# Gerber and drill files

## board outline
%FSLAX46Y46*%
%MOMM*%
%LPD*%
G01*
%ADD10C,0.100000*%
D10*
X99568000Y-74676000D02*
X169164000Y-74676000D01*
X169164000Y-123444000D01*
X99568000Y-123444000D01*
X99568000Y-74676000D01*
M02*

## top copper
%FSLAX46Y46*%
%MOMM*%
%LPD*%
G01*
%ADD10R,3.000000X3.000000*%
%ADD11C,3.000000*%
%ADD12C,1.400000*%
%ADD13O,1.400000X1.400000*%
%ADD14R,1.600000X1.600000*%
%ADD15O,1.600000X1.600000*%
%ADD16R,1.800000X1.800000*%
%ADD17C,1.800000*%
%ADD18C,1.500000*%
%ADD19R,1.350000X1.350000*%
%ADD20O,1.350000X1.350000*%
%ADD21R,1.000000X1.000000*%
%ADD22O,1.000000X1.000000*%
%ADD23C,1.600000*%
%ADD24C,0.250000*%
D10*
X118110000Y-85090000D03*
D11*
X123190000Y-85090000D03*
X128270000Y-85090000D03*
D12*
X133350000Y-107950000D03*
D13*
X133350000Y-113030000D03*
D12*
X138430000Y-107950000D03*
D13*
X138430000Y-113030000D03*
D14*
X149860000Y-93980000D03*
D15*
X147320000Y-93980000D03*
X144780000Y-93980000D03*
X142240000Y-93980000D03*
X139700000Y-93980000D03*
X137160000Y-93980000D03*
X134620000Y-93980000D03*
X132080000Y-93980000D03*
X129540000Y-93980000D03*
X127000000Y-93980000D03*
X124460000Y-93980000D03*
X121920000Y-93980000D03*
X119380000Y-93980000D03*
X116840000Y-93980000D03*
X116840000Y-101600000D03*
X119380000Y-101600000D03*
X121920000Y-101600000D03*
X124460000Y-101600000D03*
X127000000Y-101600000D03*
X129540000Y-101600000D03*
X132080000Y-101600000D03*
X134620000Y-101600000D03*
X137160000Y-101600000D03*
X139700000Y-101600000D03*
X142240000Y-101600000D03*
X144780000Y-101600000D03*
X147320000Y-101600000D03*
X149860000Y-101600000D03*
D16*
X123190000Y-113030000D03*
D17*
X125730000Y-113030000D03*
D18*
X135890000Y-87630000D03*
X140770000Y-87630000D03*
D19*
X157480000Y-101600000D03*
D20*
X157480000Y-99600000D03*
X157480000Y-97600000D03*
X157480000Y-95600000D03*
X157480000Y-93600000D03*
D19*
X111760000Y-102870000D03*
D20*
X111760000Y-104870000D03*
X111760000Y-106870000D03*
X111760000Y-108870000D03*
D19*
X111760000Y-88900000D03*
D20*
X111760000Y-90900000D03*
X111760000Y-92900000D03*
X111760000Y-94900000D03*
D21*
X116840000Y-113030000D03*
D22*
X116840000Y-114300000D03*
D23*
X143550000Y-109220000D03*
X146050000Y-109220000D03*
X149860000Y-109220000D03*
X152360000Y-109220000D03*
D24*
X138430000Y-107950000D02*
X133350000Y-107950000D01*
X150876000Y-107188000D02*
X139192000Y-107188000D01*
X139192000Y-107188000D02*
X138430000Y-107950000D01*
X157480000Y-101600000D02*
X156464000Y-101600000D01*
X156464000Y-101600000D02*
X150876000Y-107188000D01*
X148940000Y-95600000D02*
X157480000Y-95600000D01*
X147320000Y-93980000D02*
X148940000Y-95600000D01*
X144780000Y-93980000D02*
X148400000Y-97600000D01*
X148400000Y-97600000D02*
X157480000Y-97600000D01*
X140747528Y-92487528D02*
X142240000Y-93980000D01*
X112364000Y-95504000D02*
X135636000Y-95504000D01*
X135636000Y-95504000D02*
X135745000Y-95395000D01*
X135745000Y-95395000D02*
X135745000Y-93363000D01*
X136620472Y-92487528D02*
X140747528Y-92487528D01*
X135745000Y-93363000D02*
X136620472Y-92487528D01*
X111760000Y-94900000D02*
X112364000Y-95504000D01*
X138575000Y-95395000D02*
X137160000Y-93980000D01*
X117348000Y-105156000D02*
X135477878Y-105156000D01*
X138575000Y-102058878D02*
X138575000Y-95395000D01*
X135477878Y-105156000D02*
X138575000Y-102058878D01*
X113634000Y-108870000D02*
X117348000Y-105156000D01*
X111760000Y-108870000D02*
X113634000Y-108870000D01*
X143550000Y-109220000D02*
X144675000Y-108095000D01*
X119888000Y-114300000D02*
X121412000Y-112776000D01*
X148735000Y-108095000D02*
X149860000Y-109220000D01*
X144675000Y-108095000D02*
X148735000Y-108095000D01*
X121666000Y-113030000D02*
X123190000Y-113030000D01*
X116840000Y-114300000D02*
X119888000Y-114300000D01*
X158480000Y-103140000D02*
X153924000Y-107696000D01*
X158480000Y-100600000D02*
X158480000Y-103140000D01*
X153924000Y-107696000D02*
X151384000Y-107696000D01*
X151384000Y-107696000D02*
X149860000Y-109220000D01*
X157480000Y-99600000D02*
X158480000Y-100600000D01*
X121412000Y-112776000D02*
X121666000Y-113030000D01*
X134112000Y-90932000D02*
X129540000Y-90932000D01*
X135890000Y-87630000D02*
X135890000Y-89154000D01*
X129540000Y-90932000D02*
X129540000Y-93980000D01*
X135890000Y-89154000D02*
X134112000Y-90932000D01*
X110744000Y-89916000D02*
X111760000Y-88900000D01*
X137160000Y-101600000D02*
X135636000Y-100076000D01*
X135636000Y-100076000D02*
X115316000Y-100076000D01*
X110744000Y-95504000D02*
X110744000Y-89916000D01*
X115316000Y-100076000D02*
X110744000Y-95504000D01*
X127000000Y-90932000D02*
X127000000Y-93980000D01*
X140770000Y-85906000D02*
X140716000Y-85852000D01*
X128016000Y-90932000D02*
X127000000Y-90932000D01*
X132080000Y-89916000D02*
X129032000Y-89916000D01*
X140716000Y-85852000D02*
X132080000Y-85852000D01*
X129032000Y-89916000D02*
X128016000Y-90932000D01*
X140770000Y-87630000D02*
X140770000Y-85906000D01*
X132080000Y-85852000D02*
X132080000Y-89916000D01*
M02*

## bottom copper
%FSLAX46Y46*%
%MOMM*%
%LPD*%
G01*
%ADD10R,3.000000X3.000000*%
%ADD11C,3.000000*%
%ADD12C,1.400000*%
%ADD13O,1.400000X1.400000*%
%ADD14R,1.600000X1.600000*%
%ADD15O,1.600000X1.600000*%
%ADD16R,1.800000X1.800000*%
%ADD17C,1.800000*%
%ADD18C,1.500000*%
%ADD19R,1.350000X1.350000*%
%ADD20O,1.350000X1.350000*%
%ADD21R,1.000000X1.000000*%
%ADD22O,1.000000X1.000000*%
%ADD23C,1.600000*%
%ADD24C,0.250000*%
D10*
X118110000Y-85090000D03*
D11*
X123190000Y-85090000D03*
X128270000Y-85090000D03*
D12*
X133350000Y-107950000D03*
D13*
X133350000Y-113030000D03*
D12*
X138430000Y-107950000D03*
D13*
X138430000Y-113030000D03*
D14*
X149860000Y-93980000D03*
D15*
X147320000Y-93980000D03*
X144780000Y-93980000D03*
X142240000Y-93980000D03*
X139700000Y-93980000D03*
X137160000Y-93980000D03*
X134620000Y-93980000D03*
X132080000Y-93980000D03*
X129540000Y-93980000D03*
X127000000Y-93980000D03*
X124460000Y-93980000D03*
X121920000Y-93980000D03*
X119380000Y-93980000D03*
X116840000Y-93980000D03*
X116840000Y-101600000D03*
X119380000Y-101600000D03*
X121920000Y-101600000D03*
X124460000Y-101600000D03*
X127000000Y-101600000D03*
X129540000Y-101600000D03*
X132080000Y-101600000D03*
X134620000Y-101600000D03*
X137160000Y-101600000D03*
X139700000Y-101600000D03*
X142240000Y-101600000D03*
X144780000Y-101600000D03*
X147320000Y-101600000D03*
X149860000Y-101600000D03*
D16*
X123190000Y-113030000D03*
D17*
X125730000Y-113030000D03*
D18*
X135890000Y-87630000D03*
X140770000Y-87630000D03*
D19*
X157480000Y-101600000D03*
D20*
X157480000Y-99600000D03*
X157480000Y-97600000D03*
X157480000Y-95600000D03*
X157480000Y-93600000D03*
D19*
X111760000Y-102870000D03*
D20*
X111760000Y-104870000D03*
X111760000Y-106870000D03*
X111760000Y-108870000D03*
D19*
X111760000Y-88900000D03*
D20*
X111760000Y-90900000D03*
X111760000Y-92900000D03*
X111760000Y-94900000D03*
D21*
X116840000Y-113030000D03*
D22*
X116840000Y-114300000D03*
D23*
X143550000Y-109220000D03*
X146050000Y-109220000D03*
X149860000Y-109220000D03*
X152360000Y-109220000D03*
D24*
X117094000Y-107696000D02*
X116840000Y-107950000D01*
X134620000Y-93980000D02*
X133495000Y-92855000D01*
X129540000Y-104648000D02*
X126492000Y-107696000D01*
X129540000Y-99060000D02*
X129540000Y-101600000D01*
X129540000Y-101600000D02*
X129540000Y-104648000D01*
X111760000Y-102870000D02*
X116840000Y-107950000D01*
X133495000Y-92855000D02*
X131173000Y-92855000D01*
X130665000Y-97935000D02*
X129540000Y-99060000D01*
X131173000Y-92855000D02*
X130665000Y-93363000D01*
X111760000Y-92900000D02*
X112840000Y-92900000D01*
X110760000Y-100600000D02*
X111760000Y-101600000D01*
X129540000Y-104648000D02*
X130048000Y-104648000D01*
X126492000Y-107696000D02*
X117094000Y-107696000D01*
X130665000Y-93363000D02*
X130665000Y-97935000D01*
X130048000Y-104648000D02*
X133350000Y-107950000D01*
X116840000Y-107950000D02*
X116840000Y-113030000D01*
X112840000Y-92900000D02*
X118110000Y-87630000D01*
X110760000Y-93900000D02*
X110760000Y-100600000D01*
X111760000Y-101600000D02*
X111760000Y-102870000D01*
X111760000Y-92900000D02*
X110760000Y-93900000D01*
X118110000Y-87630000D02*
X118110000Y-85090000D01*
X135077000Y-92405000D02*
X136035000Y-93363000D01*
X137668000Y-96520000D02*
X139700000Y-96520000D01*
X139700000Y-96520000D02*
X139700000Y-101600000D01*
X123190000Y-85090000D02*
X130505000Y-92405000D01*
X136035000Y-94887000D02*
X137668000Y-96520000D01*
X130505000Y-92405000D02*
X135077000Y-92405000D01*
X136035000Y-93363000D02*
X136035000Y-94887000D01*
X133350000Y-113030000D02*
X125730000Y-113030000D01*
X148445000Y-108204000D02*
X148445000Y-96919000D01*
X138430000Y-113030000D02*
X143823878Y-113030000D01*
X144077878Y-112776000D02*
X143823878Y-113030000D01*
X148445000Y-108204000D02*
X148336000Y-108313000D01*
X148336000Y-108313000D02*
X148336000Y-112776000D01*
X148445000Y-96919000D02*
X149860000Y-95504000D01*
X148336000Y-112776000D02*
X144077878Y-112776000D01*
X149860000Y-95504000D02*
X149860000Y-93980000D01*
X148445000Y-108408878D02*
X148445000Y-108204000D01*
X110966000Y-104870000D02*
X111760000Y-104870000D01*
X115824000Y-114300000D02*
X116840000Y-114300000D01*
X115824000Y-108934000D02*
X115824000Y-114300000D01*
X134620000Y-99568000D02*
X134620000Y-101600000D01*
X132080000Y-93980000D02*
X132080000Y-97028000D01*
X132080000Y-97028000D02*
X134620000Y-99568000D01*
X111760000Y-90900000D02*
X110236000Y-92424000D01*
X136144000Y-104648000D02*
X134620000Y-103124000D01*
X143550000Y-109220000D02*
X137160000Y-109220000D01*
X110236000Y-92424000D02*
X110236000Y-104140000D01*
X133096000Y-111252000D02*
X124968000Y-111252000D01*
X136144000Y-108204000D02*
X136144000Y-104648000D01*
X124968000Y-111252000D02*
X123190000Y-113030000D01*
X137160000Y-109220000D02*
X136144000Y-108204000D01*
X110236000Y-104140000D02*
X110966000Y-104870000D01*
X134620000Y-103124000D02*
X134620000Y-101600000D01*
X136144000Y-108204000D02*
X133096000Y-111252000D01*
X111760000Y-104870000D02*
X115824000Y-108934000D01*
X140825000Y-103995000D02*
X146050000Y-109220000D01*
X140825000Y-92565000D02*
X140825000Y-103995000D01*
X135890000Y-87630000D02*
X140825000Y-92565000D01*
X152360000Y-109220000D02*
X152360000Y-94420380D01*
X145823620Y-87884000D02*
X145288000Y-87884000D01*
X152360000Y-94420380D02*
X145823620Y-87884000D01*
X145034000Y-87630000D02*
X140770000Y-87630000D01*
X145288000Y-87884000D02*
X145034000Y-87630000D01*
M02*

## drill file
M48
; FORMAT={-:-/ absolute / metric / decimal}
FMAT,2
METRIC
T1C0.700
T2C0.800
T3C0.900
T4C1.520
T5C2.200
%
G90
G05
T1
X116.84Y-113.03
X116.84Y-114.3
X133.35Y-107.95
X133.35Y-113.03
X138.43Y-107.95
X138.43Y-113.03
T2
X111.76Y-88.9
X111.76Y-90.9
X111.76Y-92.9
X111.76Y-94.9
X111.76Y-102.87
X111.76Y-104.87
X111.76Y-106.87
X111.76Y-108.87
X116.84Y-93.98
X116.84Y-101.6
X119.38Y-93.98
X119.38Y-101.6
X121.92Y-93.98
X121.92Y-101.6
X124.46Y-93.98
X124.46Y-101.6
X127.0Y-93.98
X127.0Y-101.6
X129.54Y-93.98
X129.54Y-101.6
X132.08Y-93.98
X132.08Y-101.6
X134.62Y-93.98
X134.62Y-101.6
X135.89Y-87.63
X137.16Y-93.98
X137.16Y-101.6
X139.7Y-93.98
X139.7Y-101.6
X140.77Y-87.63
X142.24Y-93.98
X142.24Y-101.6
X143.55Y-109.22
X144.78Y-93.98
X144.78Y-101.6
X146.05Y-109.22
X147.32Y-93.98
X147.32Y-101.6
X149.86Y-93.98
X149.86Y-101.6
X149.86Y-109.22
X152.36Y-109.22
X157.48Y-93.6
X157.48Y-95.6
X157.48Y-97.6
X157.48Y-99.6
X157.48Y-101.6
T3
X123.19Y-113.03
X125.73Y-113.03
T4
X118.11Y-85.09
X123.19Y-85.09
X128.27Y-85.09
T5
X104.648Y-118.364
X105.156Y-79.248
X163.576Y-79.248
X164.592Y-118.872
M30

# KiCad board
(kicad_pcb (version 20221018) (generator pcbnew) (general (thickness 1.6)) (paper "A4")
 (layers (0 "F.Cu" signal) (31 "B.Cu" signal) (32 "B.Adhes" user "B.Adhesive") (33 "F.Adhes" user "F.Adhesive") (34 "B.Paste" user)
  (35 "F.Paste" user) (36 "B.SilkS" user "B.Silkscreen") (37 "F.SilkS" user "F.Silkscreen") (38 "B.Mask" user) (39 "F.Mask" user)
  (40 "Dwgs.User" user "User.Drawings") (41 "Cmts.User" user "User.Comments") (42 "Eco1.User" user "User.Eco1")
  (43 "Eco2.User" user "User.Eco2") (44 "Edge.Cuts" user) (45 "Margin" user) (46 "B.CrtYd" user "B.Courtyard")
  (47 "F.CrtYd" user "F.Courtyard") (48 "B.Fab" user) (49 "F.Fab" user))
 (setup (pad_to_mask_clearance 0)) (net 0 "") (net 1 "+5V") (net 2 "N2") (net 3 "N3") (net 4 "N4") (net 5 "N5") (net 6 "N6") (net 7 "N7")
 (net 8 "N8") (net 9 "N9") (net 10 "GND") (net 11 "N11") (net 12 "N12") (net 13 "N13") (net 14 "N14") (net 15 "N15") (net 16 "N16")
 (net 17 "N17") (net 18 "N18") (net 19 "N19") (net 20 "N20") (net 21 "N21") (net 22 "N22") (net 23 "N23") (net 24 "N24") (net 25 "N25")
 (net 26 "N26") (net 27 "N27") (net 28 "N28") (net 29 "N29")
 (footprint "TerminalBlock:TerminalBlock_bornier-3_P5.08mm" (layer "F.Cu") (at 118.11 85.09)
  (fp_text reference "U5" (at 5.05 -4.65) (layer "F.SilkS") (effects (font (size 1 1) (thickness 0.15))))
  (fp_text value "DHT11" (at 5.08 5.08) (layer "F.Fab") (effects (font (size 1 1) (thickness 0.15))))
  (pad "1" thru_hole rect (at 0 0) (size 3 3) (drill 1.52) (layers "*.Cu" "*.Mask") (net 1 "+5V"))
  (pad "2" thru_hole circle (at 5.08 0) (size 3 3) (drill 1.52) (layers "*.Cu" "*.Mask") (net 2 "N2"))
  (pad "3" thru_hole circle (at 10.16 0) (size 3 3) (drill 1.52) (layers "*.Cu" "*.Mask")))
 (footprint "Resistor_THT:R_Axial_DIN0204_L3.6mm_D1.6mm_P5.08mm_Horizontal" (layer "F.Cu") (at 133.35 107.95 -90)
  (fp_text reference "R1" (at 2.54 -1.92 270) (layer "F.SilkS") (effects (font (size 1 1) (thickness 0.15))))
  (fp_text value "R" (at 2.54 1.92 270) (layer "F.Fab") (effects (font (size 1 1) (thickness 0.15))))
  (pad "1" thru_hole circle (at 0 0 270) (size 1.4 1.4) (drill 0.7) (layers "*.Cu" "*.Mask") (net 1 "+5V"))
  (pad "2" thru_hole oval (at 5.08 0 270) (size 1.4 1.4) (drill 0.7) (layers "*.Cu" "*.Mask") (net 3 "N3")))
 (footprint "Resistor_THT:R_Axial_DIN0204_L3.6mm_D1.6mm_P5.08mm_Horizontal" (layer "F.Cu") (at 138.43 107.95 -90)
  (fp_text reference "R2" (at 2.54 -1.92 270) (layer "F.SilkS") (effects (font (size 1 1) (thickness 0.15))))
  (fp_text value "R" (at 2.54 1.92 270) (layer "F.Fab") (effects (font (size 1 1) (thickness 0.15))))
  (pad "1" thru_hole circle (at 0 0 270) (size 1.4 1.4) (drill 0.7) (layers "*.Cu" "*.Mask") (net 1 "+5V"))
  (pad "2" thru_hole oval (at 5.08 0 270) (size 1.4 1.4) (drill 0.7) (layers "*.Cu" "*.Mask") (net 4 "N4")))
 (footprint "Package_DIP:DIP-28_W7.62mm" (layer "F.Cu") (at 149.86 93.98 -90)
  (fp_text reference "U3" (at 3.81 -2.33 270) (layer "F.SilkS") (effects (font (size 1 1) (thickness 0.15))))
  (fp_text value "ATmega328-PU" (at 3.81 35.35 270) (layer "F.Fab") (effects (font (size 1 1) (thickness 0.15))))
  (pad "1" thru_hole rect (at 0 0 270) (size 1.6 1.6) (drill 0.8) (layers "*.Cu" "*.Mask") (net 4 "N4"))
  (pad "2" thru_hole oval (at 0 2.54 270) (size 1.6 1.6) (drill 0.8) (layers "*.Cu" "*.Mask") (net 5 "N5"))
  (pad "3" thru_hole oval (at 0 5.08 270) (size 1.6 1.6) (drill 0.8) (layers "*.Cu" "*.Mask") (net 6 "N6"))
  (pad "4" thru_hole oval (at 0 7.62 270) (size 1.6 1.6) (drill 0.8) (layers "*.Cu" "*.Mask") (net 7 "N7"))
  (pad "5" thru_hole oval (at 0 10.16 270) (size 1.6 1.6) (drill 0.8) (layers "*.Cu" "*.Mask") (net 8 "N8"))
  (pad "6" thru_hole oval (at 0 12.7 270) (size 1.6 1.6) (drill 0.8) (layers "*.Cu" "*.Mask") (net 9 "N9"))
  (pad "7" thru_hole oval (at 0 15.24 270) (size 1.6 1.6) (drill 0.8) (layers "*.Cu" "*.Mask") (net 1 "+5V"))
  (pad "8" thru_hole oval (at 0 17.78 270) (size 1.6 1.6) (drill 0.8) (layers "*.Cu" "*.Mask") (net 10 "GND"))
  (pad "9" thru_hole oval (at 0 20.32 270) (size 1.6 1.6) (drill 0.8) (layers "*.Cu" "*.Mask") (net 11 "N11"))
  (pad "10" thru_hole oval (at 0 22.86 270) (size 1.6 1.6) (drill 0.8) (layers "*.Cu" "*.Mask") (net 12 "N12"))
  (pad "11" thru_hole oval (at 0 25.4 270) (size 1.6 1.6) (drill 0.8) (layers "*.Cu" "*.Mask") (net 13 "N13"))
  (pad "12" thru_hole oval (at 0 27.94 270) (size 1.6 1.6) (drill 0.8) (layers "*.Cu" "*.Mask") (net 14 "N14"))
  (pad "13" thru_hole oval (at 0 30.48 270) (size 1.6 1.6) (drill 0.8) (layers "*.Cu" "*.Mask") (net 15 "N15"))
  (pad "14" thru_hole oval (at 0 33.02 270) (size 1.6 1.6) (drill 0.8) (layers "*.Cu" "*.Mask") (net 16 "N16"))
  (pad "15" thru_hole oval (at 7.62 33.02 270) (size 1.6 1.6) (drill 0.8) (layers "*.Cu" "*.Mask") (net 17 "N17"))
  (pad "16" thru_hole oval (at 7.62 30.48 270) (size 1.6 1.6) (drill 0.8) (layers "*.Cu" "*.Mask") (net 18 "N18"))
  (pad "17" thru_hole oval (at 7.62 27.94 270) (size 1.6 1.6) (drill 0.8) (layers "*.Cu" "*.Mask") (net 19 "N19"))
  (pad "18" thru_hole oval (at 7.62 25.4 270) (size 1.6 1.6) (drill 0.8) (layers "*.Cu" "*.Mask") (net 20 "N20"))
  (pad "19" thru_hole oval (at 7.62 22.86 270) (size 1.6 1.6) (drill 0.8) (layers "*.Cu" "*.Mask") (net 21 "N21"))
  (pad "20" thru_hole oval (at 7.62 20.32 270) (size 1.6 1.6) (drill 0.8) (layers "*.Cu" "*.Mask") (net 1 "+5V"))
  (pad "21" thru_hole oval (at 7.62 17.78 270) (size 1.6 1.6) (drill 0.8) (layers "*.Cu" "*.Mask") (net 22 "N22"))
  (pad "22" thru_hole oval (at 7.62 15.24 270) (size 1.6 1.6) (drill 0.8) (layers "*.Cu" "*.Mask") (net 10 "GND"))
  (pad "23" thru_hole oval (at 7.62 12.7 270) (size 1.6 1.6) (drill 0.8) (layers "*.Cu" "*.Mask") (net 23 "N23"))
  (pad "24" thru_hole oval (at 7.62 10.16 270) (size 1.6 1.6) (drill 0.8) (layers "*.Cu" "*.Mask") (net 2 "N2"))
  (pad "25" thru_hole oval (at 7.62 7.62 270) (size 1.6 1.6) (drill 0.8) (layers "*.Cu" "*.Mask") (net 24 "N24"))
  (pad "26" thru_hole oval (at 7.62 5.08 270) (size 1.6 1.6) (drill 0.8) (layers "*.Cu" "*.Mask") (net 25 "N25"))
  (pad "27" thru_hole oval (at 7.62 2.54 270) (size 1.6 1.6) (drill 0.8) (layers "*.Cu" "*.Mask") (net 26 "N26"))
  (pad "28" thru_hole oval (at 7.62 0 270) (size 1.6 1.6) (drill 0.8) (layers "*.Cu" "*.Mask") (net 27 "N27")))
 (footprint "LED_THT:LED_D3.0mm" (layer "F.Cu") (at 123.19 113.03)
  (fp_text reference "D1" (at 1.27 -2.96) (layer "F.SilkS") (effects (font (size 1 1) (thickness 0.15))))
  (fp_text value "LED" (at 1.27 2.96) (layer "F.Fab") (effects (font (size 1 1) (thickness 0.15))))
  (pad "1" thru_hole rect (at 0 0) (size 1.8 1.8) (drill 0.9) (layers "*.Cu" "*.Mask") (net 10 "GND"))
  (pad "2" thru_hole circle (at 2.54 0) (size 1.8 1.8) (drill 0.9) (layers "*.Cu" "*.Mask") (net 3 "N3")))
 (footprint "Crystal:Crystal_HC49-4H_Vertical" (layer "F.Cu") (at 135.89 87.63)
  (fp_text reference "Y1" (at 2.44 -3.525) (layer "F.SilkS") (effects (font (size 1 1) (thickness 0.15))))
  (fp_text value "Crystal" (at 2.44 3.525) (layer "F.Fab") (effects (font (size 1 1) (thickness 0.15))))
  (pad "1" thru_hole circle (at 0 0) (size 1.5 1.5) (drill 0.8) (layers "*.Cu" "*.Mask") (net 11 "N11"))
  (pad "2" thru_hole circle (at 4.88 0) (size 1.5 1.5) (drill 0.8) (layers "*.Cu" "*.Mask") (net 12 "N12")))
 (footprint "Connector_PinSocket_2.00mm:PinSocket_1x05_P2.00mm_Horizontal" (layer "F.Cu") (at 157.48 101.6 180)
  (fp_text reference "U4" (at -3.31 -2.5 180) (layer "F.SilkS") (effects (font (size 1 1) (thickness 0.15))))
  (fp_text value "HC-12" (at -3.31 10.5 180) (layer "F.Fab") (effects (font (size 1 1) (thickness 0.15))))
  (pad "1" thru_hole rect (at 0 0 180) (size 1.35 1.35) (drill 0.8) (layers "*.Cu" "*.Mask") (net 1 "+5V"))
  (pad "2" thru_hole oval (at 0 2 180) (size 1.35 1.35) (drill 0.8) (layers "*.Cu" "*.Mask") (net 10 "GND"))
  (pad "3" thru_hole oval (at 0 4 180) (size 1.35 1.35) (drill 0.8) (layers "*.Cu" "*.Mask") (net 6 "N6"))
  (pad "4" thru_hole oval (at 0 6 180) (size 1.35 1.35) (drill 0.8) (layers "*.Cu" "*.Mask") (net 5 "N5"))
  (pad "5" thru_hole oval (at 0 8 180) (size 1.35 1.35) (drill 0.8) (layers "*.Cu" "*.Mask") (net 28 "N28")))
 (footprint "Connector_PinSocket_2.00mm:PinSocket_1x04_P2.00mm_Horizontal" (layer "F.Cu") (at 111.76 102.87)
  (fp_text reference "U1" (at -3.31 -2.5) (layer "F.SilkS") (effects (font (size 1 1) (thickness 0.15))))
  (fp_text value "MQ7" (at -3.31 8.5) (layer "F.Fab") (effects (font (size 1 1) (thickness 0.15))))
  (pad "1" thru_hole rect (at 0 0) (size 1.35 1.35) (drill 0.8) (layers "*.Cu" "*.Mask") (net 1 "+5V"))
  (pad "2" thru_hole oval (at 0 2) (size 1.35 1.35) (drill 0.8) (layers "*.Cu" "*.Mask") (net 10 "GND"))
  (pad "3" thru_hole oval (at 0 4) (size 1.35 1.35) (drill 0.8) (layers "*.Cu" "*.Mask") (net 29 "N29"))
  (pad "4" thru_hole oval (at 0 6) (size 1.35 1.35) (drill 0.8) (layers "*.Cu" "*.Mask") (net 9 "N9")))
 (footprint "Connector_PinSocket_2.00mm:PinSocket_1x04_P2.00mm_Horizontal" (layer "F.Cu") (at 111.76 88.9)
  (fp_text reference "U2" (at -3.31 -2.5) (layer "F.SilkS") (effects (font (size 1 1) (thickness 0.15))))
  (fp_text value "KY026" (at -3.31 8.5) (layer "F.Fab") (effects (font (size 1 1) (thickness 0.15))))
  (pad "1" thru_hole rect (at 0 0) (size 1.35 1.35) (drill 0.8) (layers "*.Cu" "*.Mask") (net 23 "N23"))
  (pad "2" thru_hole oval (at 0 2) (size 1.35 1.35) (drill 0.8) (layers "*.Cu" "*.Mask") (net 10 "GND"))
  (pad "3" thru_hole oval (at 0 4) (size 1.35 1.35) (drill 0.8) (layers "*.Cu" "*.Mask") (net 1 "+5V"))
  (pad "4" thru_hole oval (at 0 6) (size 1.35 1.35) (drill 0.8) (layers "*.Cu" "*.Mask") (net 7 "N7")))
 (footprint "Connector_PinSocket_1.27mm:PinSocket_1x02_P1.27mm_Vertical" (layer "F.Cu") (at 116.84 113.03)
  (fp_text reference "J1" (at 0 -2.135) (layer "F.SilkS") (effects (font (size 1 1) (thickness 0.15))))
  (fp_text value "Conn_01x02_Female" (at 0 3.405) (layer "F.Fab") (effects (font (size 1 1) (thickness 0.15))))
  (pad "1" thru_hole rect (at 0 0) (size 1 1) (drill 0.7) (layers "*.Cu" "*.Mask") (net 1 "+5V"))
  (pad "2" thru_hole oval (at 0 1.27) (size 1 1) (drill 0.7) (layers "*.Cu" "*.Mask") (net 10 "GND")))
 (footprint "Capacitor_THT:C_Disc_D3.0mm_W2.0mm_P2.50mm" (layer "F.Cu") (at 143.55 109.22)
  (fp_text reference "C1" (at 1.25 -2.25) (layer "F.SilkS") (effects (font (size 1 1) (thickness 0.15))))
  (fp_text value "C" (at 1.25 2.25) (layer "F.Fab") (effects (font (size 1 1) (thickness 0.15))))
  (pad "1" thru_hole circle (at 0 0) (size 1.6 1.6) (drill 0.8) (layers "*.Cu" "*.Mask") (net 10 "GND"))
  (pad "2" thru_hole circle (at 2.5 0) (size 1.6 1.6) (drill 0.8) (layers "*.Cu" "*.Mask") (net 11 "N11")))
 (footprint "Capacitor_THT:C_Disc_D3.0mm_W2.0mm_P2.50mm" (layer "F.Cu") (at 149.86 109.22)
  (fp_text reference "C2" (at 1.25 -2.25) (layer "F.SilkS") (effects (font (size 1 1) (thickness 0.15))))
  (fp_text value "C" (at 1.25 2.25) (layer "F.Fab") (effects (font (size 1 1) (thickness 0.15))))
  (pad "1" thru_hole circle (at 0 0) (size 1.6 1.6) (drill 0.8) (layers "*.Cu" "*.Mask") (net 10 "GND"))
  (pad "2" thru_hole circle (at 2.5 0) (size 1.6 1.6) (drill 0.8) (layers "*.Cu" "*.Mask") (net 12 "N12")))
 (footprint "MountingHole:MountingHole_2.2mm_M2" (layer "F.Cu") (at 104.648 118.364)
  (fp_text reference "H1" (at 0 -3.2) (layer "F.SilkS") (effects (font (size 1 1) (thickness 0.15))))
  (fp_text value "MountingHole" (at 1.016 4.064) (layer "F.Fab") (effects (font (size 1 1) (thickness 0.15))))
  (pad "" np_thru_hole circle (at 0 0) (size 2.2 2.2) (drill 2.2) (layers "*.Cu" "*.Mask")))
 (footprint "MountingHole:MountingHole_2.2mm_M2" (layer "F.Cu") (at 164.592 118.872)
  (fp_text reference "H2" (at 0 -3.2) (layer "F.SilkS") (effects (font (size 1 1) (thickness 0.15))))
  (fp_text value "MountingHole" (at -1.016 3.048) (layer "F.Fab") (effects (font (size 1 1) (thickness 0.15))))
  (pad "" np_thru_hole circle (at 0 0) (size 2.2 2.2) (drill 2.2) (layers "*.Cu" "*.Mask")))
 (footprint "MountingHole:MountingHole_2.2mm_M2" (layer "F.Cu") (at 105.156 79.248)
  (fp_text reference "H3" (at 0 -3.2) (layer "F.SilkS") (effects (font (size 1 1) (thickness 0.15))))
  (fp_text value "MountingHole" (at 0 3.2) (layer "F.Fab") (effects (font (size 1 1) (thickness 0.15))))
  (pad "" np_thru_hole circle (at 0 0) (size 2.2 2.2) (drill 2.2) (layers "*.Cu" "*.Mask")))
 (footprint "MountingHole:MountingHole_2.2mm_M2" (layer "F.Cu") (at 163.576 79.248)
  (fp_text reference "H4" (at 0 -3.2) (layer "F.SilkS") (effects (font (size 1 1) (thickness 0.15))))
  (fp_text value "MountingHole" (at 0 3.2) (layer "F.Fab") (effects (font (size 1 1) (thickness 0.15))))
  (pad "" np_thru_hole circle (at 0 0) (size 2.2 2.2) (drill 2.2) (layers "*.Cu" "*.Mask")))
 (gr_rect (start 99.568 74.676) (end 169.164 123.444) (stroke (width 0.1) (type default)) (fill none) (layer "Edge.Cuts"))
 (segment (start 138.43 107.95) (end 133.35 107.95) (width 0.25) (layer "F.Cu") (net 1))
 (segment (start 150.876 107.188) (end 139.192 107.188) (width 0.25) (layer "F.Cu") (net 1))
 (segment (start 139.192 107.188) (end 138.43 107.95) (width 0.25) (layer "F.Cu") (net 1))
 (segment (start 157.48 101.6) (end 156.464 101.6) (width 0.25) (layer "F.Cu") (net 1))
 (segment (start 156.464 101.6) (end 150.876 107.188) (width 0.25) (layer "F.Cu") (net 1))
 (segment (start 117.094 107.696) (end 116.84 107.95) (width 0.25) (layer "B.Cu") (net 1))
 (segment (start 134.62 93.98) (end 133.495 92.855) (width 0.25) (layer "B.Cu") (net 1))
 (segment (start 129.54 104.648) (end 126.492 107.696) (width 0.25) (layer "B.Cu") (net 1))
 (segment (start 129.54 99.06) (end 129.54 101.6) (width 0.25) (layer "B.Cu") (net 1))
 (segment (start 129.54 101.6) (end 129.54 104.648) (width 0.25) (layer "B.Cu") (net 1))
 (segment (start 111.76 102.87) (end 116.84 107.95) (width 0.25) (layer "B.Cu") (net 1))
 (segment (start 133.495 92.855) (end 131.173 92.855) (width 0.25) (layer "B.Cu") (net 1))
 (segment (start 130.665 97.935) (end 129.54 99.06) (width 0.25) (layer "B.Cu") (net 1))
 (segment (start 131.173 92.855) (end 130.665 93.363) (width 0.25) (layer "B.Cu") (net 1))
 (segment (start 111.76 92.9) (end 112.84 92.9) (width 0.25) (layer "B.Cu") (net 1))
 (segment (start 110.76 100.6) (end 111.76 101.6) (width 0.25) (layer "B.Cu") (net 1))
 (segment (start 129.54 104.648) (end 130.048 104.648) (width 0.25) (layer "B.Cu") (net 1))
 (segment (start 126.492 107.696) (end 117.094 107.696) (width 0.25) (layer "B.Cu") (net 1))
 (segment (start 130.665 93.363) (end 130.665 97.935) (width 0.25) (layer "B.Cu") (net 1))
 (segment (start 130.048 104.648) (end 133.35 107.95) (width 0.25) (layer "B.Cu") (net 1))
 (segment (start 116.84 107.95) (end 116.84 113.03) (width 0.25) (layer "B.Cu") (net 1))
 (segment (start 112.84 92.9) (end 118.11 87.63) (width 0.25) (layer "B.Cu") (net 1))
 (segment (start 110.76 93.9) (end 110.76 100.6) (width 0.25) (layer "B.Cu") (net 1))
 (segment (start 111.76 101.6) (end 111.76 102.87) (width 0.25) (layer "B.Cu") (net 1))
 (segment (start 111.76 92.9) (end 110.76 93.9) (width 0.25) (layer "B.Cu") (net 1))
 (segment (start 118.11 87.63) (end 118.11 85.09) (width 0.25) (layer "B.Cu") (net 1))
 (segment (start 135.077 92.405) (end 136.035 93.363) (width 0.25) (layer "B.Cu") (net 2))
 (segment (start 137.668 96.52) (end 139.7 96.52) (width 0.25) (layer "B.Cu") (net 2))
 (segment (start 139.7 96.52) (end 139.7 101.6) (width 0.25) (layer "B.Cu") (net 2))
 (segment (start 123.19 85.09) (end 130.505 92.405) (width 0.25) (layer "B.Cu") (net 2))
 (segment (start 136.035 94.887) (end 137.668 96.52) (width 0.25) (layer "B.Cu") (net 2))
 (segment (start 130.505 92.405) (end 135.077 92.405) (width 0.25) (layer "B.Cu") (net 2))
 (segment (start 136.035 93.363) (end 136.035 94.887) (width 0.25) (layer "B.Cu") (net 2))
 (segment (start 133.35 113.03) (end 125.73 113.03) (width 0.25) (layer "B.Cu") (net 3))
 (segment (start 148.445 108.204) (end 148.445 96.919) (width 0.25) (layer "B.Cu") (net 4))
 (segment (start 138.43 113.03) (end 143.823878 113.03) (width 0.25) (layer "B.Cu") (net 4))
 (segment (start 144.077878 112.776) (end 143.823878 113.03) (width 0.25) (layer "B.Cu") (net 4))
 (segment (start 148.445 108.204) (end 148.336 108.313) (width 0.25) (layer "B.Cu") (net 4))
 (segment (start 148.336 108.313) (end 148.336 112.776) (width 0.25) (layer "B.Cu") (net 4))
 (segment (start 148.445 96.919) (end 149.86 95.504) (width 0.25) (layer "B.Cu") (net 4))
 (segment (start 148.336 112.776) (end 144.077878 112.776) (width 0.25) (layer "B.Cu") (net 4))
 (segment (start 149.86 95.504) (end 149.86 93.98) (width 0.25) (layer "B.Cu") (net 4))
 (segment (start 148.445 108.408878) (end 148.445 108.204) (width 0.25) (layer "B.Cu") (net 4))
 (segment (start 148.94 95.6) (end 157.48 95.6) (width 0.25) (layer "F.Cu") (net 5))
 (segment (start 147.32 93.98) (end 148.94 95.6) (width 0.25) (layer "F.Cu") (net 5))
 (segment (start 144.78 93.98) (end 148.4 97.6) (width 0.25) (layer "F.Cu") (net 6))
 (segment (start 148.4 97.6) (end 157.48 97.6) (width 0.25) (layer "F.Cu") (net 6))
 (segment (start 140.747528 92.487528) (end 142.24 93.98) (width 0.25) (layer "F.Cu") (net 7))
 (segment (start 112.364 95.504) (end 135.636 95.504) (width 0.25) (layer "F.Cu") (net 7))
 (segment (start 135.636 95.504) (end 135.745 95.395) (width 0.25) (layer "F.Cu") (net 7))
 (segment (start 135.745 95.395) (end 135.745 93.363) (width 0.25) (layer "F.Cu") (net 7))
 (segment (start 136.620472 92.487528) (end 140.747528 92.487528) (width 0.25) (layer "F.Cu") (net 7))
 (segment (start 135.745 93.363) (end 136.620472 92.487528) (width 0.25) (layer "F.Cu") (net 7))
 (segment (start 111.76 94.9) (end 112.364 95.504) (width 0.25) (layer "F.Cu") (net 7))
 (segment (start 138.575 95.395) (end 137.16 93.98) (width 0.25) (layer "F.Cu") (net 9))
 (segment (start 117.348 105.156) (end 135.477878 105.156) (width 0.25) (layer "F.Cu") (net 9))
 (segment (start 138.575 102.058878) (end 138.575 95.395) (width 0.25) (layer "F.Cu") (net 9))
 (segment (start 135.477878 105.156) (end 138.575 102.058878) (width 0.25) (layer "F.Cu") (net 9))
 (segment (start 113.634 108.87) (end 117.348 105.156) (width 0.25) (layer "F.Cu") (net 9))
 (segment (start 111.76 108.87) (end 113.634 108.87) (width 0.25) (layer "F.Cu") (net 9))
 (segment (start 143.55 109.22) (end 144.675 108.095) (width 0.25) (layer "F.Cu") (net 10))
 (segment (start 119.888 114.3) (end 121.412 112.776) (width 0.25) (layer "F.Cu") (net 10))
 (segment (start 148.735 108.095) (end 149.86 109.22) (width 0.25) (layer "F.Cu") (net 10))
 (segment (start 144.675 108.095) (end 148.735 108.095) (width 0.25) (layer "F.Cu") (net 10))
 (segment (start 121.666 113.03) (end 123.19 113.03) (width 0.25) (layer "F.Cu") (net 10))
 (segment (start 116.84 114.3) (end 119.888 114.3) (width 0.25) (layer "F.Cu") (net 10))
 (segment (start 158.48 103.14) (end 153.924 107.696) (width 0.25) (layer "F.Cu") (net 10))
 (segment (start 158.48 100.6) (end 158.48 103.14) (width 0.25) (layer "F.Cu") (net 10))
 (segment (start 153.924 107.696) (end 151.384 107.696) (width 0.25) (layer "F.Cu") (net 10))
 (segment (start 151.384 107.696) (end 149.86 109.22) (width 0.25) (layer "F.Cu") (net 10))
 (segment (start 157.48 99.6) (end 158.48 100.6) (width 0.25) (layer "F.Cu") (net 10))
 (segment (start 121.412 112.776) (end 121.666 113.03) (width 0.25) (layer "F.Cu") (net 10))
 (segment (start 110.966 104.87) (end 111.76 104.87) (width 0.25) (layer "B.Cu") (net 10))
 (segment (start 115.824 114.3) (end 116.84 114.3) (width 0.25) (layer "B.Cu") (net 10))
 (segment (start 115.824 108.934) (end 115.824 114.3) (width 0.25) (layer "B.Cu") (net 10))
 (segment (start 134.62 99.568) (end 134.62 101.6) (width 0.25) (layer "B.Cu") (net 10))
 (segment (start 132.08 93.98) (end 132.08 97.028) (width 0.25) (layer "B.Cu") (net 10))
 (segment (start 132.08 97.028) (end 134.62 99.568) (width 0.25) (layer "B.Cu") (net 10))
 (segment (start 111.76 90.9) (end 110.236 92.424) (width 0.25) (layer "B.Cu") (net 10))
 (segment (start 136.144 104.648) (end 134.62 103.124) (width 0.25) (layer "B.Cu") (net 10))
 (segment (start 143.55 109.22) (end 137.16 109.22) (width 0.25) (layer "B.Cu") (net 10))
 (segment (start 110.236 92.424) (end 110.236 104.14) (width 0.25) (layer "B.Cu") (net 10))
 (segment (start 133.096 111.252) (end 124.968 111.252) (width 0.25) (layer "B.Cu") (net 10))
 (segment (start 136.144 108.204) (end 136.144 104.648) (width 0.25) (layer "B.Cu") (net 10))
 (segment (start 124.968 111.252) (end 123.19 113.03) (width 0.25) (layer "B.Cu") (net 10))
 (segment (start 137.16 109.22) (end 136.144 108.204) (width 0.25) (layer "B.Cu") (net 10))
 (segment (start 110.236 104.14) (end 110.966 104.87) (width 0.25) (layer "B.Cu") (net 10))
 (segment (start 134.62 103.124) (end 134.62 101.6) (width 0.25) (layer "B.Cu") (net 10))
 (segment (start 136.144 108.204) (end 133.096 111.252) (width 0.25) (layer "B.Cu") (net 10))
 (segment (start 111.76 104.87) (end 115.824 108.934) (width 0.25) (layer "B.Cu") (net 10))
 (segment (start 134.112 90.932) (end 129.54 90.932) (width 0.25) (layer "F.Cu") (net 11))
 (segment (start 135.89 87.63) (end 135.89 89.154) (width 0.25) (layer "F.Cu") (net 11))
 (segment (start 129.54 90.932) (end 129.54 93.98) (width 0.25) (layer "F.Cu") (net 11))
 (segment (start 135.89 89.154) (end 134.112 90.932) (width 0.25) (layer "F.Cu") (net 11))
 (segment (start 140.825 103.995) (end 146.05 109.22) (width 0.25) (layer "B.Cu") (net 11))
 (segment (start 140.825 92.565) (end 140.825 103.995) (width 0.25) (layer "B.Cu") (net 11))
 (segment (start 135.89 87.63) (end 140.825 92.565) (width 0.25) (layer "B.Cu") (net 11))
 (segment (start 110.744 89.916) (end 111.76 88.9) (width 0.25) (layer "F.Cu") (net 23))
 (segment (start 137.16 101.6) (end 135.636 100.076) (width 0.25) (layer "F.Cu") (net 23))
 (segment (start 135.636 100.076) (end 115.316 100.076) (width 0.25) (layer "F.Cu") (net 23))
 (segment (start 110.744 95.504) (end 110.744 89.916) (width 0.25) (layer "F.Cu") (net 23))
 (segment (start 115.316 100.076) (end 110.744 95.504) (width 0.25) (layer "F.Cu") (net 23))
 (segment (start 127 90.932) (end 127 93.98) (width 0.25) (layer "F.Cu") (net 12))
 (segment (start 140.77 85.906) (end 140.716 85.852) (width 0.25) (layer "F.Cu") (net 12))
 (segment (start 128.016 90.932) (end 127 90.932) (width 0.25) (layer "F.Cu") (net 12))
 (segment (start 132.08 89.916) (end 129.032 89.916) (width 0.25) (layer "F.Cu") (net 12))
 (segment (start 140.716 85.852) (end 132.08 85.852) (width 0.25) (layer "F.Cu") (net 12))
 (segment (start 129.032 89.916) (end 128.016 90.932) (width 0.25) (layer "F.Cu") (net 12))
 (segment (start 140.77 87.63) (end 140.77 85.906) (width 0.25) (layer "F.Cu") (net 12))
 (segment (start 132.08 85.852) (end 132.08 89.916) (width 0.25) (layer "F.Cu") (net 12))
 (segment (start 152.36 109.22) (end 152.36 94.42038) (width 0.25) (layer "B.Cu") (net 12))
 (segment (start 145.82362 87.884) (end 145.288 87.884) (width 0.25) (layer "B.Cu") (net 12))
 (segment (start 152.36 94.42038) (end 145.82362 87.884) (width 0.25) (layer "B.Cu") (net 12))
 (segment (start 145.034 87.63) (end 140.77 87.63) (width 0.25) (layer "B.Cu") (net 12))
 (segment (start 145.288 87.884) (end 145.034 87.63) (width 0.25) (layer "B.Cu") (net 12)))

